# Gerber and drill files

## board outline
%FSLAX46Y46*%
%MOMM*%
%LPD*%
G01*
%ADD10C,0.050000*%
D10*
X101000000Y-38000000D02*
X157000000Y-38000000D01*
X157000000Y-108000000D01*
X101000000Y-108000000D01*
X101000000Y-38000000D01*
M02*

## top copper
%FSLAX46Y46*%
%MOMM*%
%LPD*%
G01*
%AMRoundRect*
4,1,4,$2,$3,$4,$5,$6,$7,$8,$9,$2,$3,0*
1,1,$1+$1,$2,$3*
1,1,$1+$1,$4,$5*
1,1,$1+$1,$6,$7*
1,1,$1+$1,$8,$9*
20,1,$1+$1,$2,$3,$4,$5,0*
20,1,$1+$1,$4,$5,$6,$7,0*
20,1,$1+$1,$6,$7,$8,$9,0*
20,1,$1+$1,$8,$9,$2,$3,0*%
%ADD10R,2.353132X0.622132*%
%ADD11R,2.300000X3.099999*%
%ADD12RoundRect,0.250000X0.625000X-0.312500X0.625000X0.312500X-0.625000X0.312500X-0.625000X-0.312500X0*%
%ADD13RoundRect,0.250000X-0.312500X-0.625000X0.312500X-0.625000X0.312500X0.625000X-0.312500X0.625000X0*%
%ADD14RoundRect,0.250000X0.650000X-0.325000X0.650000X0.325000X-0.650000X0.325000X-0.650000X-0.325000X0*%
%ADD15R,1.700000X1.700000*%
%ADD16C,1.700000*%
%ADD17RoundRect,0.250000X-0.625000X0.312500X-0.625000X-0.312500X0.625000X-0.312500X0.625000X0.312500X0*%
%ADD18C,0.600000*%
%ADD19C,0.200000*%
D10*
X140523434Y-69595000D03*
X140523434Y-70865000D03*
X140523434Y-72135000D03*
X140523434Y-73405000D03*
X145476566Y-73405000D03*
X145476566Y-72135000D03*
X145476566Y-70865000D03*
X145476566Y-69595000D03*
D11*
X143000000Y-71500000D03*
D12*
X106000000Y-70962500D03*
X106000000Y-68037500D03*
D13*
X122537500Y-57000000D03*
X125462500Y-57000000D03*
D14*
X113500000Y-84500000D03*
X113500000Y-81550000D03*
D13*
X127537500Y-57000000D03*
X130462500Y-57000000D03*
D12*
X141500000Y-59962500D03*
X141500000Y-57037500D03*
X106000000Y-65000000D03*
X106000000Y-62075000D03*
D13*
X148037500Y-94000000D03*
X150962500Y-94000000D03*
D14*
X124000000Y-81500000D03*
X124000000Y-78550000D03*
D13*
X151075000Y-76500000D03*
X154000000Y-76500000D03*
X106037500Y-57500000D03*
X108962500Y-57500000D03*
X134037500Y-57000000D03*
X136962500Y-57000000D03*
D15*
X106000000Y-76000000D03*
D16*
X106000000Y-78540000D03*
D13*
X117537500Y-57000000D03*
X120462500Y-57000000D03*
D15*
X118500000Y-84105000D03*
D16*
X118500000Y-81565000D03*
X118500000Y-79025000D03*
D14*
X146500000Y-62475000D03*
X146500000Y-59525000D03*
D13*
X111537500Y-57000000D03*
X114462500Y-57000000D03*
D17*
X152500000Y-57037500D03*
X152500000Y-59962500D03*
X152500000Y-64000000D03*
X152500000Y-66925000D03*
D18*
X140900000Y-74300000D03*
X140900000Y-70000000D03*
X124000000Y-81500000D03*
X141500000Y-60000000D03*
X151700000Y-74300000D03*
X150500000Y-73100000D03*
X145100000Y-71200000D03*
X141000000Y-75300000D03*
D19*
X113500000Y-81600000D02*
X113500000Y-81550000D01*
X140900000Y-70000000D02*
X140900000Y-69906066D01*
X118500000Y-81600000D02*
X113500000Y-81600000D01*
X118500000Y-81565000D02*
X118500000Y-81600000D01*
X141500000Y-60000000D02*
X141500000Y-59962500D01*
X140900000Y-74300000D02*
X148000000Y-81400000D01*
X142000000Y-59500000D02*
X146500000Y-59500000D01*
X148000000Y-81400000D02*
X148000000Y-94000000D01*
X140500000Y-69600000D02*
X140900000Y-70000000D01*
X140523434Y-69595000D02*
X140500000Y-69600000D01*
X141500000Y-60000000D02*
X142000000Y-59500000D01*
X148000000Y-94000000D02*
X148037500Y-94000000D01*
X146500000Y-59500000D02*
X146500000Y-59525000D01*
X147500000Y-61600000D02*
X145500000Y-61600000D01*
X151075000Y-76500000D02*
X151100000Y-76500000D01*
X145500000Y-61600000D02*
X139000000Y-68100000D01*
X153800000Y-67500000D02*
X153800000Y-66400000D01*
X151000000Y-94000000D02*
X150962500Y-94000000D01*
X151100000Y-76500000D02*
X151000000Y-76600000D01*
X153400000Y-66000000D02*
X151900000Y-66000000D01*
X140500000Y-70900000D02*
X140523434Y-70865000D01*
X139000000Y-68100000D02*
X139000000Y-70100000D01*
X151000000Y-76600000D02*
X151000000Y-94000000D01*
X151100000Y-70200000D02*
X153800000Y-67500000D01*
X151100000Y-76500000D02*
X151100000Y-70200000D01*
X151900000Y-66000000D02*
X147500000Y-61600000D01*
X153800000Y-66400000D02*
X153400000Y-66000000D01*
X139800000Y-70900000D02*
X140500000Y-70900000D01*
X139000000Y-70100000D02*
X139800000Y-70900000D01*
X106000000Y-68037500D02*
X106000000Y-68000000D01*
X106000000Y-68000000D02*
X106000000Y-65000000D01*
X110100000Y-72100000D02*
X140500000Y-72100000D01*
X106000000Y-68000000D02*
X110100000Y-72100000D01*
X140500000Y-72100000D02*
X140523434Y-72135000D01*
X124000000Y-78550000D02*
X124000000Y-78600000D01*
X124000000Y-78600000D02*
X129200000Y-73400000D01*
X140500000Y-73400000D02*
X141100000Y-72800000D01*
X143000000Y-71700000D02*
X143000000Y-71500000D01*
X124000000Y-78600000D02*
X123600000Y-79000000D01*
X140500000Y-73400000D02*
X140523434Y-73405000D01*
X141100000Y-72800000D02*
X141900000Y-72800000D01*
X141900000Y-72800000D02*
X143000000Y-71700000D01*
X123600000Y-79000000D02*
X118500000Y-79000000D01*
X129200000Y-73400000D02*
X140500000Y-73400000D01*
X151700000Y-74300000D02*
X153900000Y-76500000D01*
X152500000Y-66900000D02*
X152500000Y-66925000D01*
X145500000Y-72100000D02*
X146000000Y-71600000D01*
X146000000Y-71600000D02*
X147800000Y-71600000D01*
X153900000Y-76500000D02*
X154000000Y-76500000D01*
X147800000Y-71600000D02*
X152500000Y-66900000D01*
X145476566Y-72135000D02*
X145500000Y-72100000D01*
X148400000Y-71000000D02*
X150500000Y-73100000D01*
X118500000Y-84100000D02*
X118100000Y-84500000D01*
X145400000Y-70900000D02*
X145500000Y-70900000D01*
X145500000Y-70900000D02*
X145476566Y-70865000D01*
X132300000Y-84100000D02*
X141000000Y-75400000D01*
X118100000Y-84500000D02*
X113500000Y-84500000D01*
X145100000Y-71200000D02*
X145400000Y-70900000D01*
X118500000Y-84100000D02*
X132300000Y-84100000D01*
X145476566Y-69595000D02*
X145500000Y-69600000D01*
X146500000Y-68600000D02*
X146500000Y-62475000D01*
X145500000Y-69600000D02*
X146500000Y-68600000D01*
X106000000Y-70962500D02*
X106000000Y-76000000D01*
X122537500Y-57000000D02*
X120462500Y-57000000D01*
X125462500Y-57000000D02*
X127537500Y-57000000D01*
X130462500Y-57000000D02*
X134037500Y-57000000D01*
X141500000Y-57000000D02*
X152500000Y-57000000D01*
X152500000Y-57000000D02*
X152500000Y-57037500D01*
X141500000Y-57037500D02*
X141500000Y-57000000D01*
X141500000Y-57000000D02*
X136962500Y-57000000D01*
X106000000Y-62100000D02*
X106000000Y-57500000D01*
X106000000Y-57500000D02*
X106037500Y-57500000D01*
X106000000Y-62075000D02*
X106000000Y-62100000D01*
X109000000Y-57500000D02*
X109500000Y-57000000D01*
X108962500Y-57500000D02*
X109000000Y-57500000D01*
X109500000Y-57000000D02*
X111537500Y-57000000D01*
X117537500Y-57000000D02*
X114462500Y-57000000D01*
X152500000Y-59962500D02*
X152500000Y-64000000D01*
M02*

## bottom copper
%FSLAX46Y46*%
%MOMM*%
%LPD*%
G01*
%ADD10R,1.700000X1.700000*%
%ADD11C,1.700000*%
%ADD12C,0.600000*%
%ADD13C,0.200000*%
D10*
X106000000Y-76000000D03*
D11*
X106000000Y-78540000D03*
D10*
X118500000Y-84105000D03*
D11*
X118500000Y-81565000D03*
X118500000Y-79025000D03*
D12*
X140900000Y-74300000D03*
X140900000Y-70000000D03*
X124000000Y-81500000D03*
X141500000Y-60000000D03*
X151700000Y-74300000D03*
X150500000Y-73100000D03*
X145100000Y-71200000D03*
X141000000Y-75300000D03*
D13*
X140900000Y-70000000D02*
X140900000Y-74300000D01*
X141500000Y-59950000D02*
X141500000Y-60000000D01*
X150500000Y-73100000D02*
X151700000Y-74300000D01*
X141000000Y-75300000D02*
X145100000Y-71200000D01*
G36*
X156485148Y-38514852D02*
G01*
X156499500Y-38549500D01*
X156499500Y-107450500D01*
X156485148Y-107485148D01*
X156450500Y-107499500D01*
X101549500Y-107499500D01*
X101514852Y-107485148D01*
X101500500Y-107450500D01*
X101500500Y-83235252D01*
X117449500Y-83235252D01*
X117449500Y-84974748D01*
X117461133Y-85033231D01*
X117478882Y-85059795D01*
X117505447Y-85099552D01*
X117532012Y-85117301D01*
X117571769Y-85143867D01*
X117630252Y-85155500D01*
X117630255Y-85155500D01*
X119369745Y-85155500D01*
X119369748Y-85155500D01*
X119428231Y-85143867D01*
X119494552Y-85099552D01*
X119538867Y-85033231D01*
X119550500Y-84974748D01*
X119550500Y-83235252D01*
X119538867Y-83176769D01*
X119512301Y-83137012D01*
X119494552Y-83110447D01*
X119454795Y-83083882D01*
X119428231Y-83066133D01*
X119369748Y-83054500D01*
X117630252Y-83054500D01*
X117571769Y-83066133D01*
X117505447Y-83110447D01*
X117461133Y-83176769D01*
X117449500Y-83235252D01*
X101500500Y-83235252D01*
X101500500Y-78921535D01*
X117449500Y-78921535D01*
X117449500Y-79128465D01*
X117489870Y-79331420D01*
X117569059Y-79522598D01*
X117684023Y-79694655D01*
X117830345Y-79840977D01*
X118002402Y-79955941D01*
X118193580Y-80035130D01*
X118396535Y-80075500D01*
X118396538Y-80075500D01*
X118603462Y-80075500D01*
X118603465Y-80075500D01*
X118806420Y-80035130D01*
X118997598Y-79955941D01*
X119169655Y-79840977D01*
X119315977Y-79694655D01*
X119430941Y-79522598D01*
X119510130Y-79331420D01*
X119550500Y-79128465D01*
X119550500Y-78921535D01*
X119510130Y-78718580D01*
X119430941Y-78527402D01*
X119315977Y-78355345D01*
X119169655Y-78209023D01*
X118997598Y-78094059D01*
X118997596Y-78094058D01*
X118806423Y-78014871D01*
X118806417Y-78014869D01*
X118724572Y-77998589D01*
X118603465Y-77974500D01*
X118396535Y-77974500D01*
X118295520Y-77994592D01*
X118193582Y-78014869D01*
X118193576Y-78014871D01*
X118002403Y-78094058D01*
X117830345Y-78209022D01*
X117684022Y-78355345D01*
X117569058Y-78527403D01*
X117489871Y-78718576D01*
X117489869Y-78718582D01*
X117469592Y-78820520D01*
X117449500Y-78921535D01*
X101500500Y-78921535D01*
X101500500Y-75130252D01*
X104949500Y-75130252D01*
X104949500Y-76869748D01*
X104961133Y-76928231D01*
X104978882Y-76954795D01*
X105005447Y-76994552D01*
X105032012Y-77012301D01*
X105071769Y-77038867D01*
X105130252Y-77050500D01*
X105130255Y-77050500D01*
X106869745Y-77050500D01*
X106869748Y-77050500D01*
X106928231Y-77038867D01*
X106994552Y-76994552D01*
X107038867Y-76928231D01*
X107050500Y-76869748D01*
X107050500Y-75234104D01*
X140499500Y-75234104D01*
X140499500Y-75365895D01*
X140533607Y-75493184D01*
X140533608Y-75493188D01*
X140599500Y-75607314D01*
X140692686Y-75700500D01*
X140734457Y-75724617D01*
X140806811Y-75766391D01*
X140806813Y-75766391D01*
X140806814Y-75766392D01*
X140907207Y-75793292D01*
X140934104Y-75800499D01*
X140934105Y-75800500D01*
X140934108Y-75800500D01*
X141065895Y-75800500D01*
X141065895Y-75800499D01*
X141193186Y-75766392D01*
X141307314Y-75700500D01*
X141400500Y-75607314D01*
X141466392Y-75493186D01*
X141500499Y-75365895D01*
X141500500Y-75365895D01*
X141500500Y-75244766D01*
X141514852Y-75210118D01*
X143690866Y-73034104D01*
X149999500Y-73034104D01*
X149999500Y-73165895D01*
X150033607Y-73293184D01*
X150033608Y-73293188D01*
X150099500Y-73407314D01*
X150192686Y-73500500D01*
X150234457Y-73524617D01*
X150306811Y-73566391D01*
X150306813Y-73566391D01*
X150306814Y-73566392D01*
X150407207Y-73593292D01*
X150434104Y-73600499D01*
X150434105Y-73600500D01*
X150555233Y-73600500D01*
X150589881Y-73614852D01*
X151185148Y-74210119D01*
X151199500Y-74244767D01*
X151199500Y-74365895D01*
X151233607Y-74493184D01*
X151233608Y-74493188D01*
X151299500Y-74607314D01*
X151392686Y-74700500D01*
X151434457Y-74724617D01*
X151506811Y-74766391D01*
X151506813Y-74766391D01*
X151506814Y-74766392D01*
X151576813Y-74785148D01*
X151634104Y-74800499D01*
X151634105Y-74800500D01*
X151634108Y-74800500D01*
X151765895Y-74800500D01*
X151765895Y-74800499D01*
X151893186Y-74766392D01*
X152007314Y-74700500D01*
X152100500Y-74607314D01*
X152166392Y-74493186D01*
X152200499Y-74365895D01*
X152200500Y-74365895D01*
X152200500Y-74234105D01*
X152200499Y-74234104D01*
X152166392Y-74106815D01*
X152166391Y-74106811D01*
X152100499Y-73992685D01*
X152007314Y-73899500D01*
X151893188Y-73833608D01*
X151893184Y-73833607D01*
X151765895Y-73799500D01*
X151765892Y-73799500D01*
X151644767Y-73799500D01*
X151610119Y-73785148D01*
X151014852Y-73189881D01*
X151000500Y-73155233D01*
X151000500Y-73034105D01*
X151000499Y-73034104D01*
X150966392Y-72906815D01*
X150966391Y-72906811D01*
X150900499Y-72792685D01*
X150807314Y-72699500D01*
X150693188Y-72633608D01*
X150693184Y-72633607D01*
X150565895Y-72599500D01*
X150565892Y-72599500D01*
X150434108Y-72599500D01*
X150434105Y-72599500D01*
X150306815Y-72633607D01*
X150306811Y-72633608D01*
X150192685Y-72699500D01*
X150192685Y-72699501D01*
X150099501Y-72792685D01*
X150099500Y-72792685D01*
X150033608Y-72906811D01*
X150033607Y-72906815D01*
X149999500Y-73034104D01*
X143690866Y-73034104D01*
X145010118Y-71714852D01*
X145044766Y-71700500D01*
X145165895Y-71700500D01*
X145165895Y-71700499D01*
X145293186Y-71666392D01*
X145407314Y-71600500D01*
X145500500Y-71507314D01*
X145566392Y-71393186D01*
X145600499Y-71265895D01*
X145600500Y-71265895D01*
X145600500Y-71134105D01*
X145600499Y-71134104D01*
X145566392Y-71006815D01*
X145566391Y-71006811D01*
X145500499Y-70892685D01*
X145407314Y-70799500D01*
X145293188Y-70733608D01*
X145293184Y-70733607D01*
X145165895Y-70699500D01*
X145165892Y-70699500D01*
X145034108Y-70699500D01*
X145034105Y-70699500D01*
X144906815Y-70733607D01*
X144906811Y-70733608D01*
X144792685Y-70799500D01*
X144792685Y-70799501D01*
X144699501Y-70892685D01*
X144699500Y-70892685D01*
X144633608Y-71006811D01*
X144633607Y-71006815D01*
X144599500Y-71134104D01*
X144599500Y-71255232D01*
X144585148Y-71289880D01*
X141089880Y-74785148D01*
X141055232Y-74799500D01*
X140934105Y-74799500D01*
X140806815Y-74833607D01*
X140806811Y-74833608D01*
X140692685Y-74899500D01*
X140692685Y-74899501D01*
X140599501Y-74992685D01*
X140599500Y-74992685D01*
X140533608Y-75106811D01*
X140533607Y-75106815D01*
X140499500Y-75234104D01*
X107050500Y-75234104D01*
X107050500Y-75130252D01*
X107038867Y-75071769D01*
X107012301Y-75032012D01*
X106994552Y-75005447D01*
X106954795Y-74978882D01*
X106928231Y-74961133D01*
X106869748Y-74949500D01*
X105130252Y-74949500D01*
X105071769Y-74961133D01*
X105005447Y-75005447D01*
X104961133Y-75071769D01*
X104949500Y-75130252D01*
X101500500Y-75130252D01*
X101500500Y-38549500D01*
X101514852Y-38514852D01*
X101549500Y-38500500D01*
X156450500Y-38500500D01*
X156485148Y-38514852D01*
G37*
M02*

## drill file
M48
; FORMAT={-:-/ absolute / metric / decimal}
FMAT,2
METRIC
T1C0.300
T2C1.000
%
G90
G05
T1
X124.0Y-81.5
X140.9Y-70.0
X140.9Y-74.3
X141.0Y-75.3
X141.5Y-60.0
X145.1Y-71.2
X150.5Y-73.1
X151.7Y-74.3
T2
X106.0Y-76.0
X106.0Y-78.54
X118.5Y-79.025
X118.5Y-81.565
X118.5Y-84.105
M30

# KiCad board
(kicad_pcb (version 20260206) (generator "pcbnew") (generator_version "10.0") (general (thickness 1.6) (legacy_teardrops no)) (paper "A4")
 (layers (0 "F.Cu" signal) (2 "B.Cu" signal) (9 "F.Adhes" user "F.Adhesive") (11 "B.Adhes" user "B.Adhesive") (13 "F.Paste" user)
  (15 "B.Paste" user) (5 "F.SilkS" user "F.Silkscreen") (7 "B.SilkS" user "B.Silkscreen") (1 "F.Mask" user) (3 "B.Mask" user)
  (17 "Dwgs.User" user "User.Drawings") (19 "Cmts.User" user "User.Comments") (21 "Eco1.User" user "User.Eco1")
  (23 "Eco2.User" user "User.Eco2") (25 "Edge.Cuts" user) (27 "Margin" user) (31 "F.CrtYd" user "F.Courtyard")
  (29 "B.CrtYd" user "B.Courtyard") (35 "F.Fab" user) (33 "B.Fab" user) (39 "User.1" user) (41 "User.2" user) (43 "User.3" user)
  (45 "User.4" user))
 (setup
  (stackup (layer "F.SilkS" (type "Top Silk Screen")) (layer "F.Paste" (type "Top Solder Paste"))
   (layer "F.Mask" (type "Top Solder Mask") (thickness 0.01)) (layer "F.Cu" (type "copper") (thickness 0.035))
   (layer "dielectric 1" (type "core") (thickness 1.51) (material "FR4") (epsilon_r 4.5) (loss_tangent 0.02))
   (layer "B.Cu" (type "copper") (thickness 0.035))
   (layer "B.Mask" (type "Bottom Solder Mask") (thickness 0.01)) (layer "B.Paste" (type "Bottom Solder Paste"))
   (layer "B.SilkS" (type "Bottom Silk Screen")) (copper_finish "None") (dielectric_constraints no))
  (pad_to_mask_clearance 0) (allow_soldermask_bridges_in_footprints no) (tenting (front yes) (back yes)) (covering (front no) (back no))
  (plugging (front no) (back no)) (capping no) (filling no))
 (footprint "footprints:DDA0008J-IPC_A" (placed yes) (layer "F.Cu") (at 143 71.5)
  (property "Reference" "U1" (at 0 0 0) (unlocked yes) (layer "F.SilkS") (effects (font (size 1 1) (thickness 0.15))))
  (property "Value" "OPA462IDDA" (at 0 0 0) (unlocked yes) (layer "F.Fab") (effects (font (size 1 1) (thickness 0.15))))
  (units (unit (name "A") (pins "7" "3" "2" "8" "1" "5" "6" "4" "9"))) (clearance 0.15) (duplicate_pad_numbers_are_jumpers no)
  (pad "1" smd rect (at -2.476566 -1.905) (size 2.353132 0.622132) (layers "F.Cu" "F.Mask" "F.Paste") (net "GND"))
  (pad "2" smd rect (at -2.476566 -0.635) (size 2.353132 0.622132) (layers "F.Cu" "F.Mask" "F.Paste") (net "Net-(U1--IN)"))
  (pad "3" smd rect (at -2.476566 0.635) (size 2.353132 0.622132) (layers "F.Cu" "F.Mask" "F.Paste") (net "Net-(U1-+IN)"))
  (pad "4" smd rect (at -2.476566 1.905) (size 2.353132 0.622132) (layers "F.Cu" "F.Mask" "F.Paste") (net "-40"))
  (pad "5" smd rect (at 2.476566 1.905) (size 2.353132 0.622132) (layers "F.Cu" "F.Mask" "F.Paste")
   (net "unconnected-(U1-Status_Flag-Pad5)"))
  (pad "6" smd rect (at 2.476566 0.635) (size 2.353132 0.622132) (layers "F.Cu" "F.Mask" "F.Paste") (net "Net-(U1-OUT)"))
  (pad "7" smd rect (at 2.476566 -0.635) (size 2.353132 0.622132) (layers "F.Cu" "F.Mask" "F.Paste") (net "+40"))
  (pad "8" smd rect (at 2.476566 -1.905) (size 2.353132 0.622132) (layers "F.Cu" "F.Mask" "F.Paste") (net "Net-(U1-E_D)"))
  (pad "9" smd rect (at 0 0) (size 2.3 3.099999) (layers "F.Cu" "F.Mask") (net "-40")))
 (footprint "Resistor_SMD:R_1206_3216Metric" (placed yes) (layer "F.Cu") (at 106 69.5 90)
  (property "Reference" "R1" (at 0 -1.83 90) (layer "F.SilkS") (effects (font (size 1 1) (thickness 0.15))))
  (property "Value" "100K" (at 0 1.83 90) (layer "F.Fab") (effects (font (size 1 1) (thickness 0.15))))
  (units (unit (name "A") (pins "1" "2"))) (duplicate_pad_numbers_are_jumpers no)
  (pad "1" smd roundrect (at -1.4625 0 90) (size 1.125 1.75) (layers "F.Cu" "F.Mask" "F.Paste") (roundrect_rratio 0.222222)
   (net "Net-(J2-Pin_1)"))
  (pad "2" smd roundrect (at 1.4625 0 90) (size 1.125 1.75) (layers "F.Cu" "F.Mask" "F.Paste") (roundrect_rratio 0.222222)
   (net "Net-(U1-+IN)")))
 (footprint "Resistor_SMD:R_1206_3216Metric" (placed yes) (layer "F.Cu") (at 124 57)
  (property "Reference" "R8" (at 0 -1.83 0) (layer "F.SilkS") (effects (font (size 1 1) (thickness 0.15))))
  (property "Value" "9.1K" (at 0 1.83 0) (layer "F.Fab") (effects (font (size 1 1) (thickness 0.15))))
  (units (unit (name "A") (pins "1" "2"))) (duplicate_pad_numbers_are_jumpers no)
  (pad "1" smd roundrect (at -1.4625 0) (size 1.125 1.75) (layers "F.Cu" "F.Mask" "F.Paste") (roundrect_rratio 0.222222)
   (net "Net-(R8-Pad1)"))
  (pad "2" smd roundrect (at 1.4625 0) (size 1.125 1.75) (layers "F.Cu" "F.Mask" "F.Paste") (roundrect_rratio 0.222222)
   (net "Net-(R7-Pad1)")))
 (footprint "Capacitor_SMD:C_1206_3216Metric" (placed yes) (layer "F.Cu") (at 113.5 83.025 90)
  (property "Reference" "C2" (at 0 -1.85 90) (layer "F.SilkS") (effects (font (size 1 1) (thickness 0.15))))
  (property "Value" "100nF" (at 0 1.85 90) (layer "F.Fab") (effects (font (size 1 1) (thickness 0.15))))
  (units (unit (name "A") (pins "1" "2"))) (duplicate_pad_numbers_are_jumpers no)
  (pad "1" smd roundrect (at -1.475 0 90) (size 1.15 1.8) (layers "F.Cu" "F.Mask" "F.Paste") (roundrect_rratio 0.217391) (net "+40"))
  (pad "2" smd roundrect (at 1.475 0 90) (size 1.15 1.8) (layers "F.Cu" "F.Mask" "F.Paste") (roundrect_rratio 0.217391) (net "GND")))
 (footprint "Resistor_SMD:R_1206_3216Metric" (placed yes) (layer "F.Cu") (at 129 57)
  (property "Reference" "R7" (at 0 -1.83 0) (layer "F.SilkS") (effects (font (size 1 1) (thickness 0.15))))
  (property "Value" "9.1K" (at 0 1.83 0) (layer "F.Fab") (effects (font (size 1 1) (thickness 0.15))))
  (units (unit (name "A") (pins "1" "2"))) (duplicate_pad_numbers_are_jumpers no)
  (pad "1" smd roundrect (at -1.4625 0) (size 1.125 1.75) (layers "F.Cu" "F.Mask" "F.Paste") (roundrect_rratio 0.222222)
   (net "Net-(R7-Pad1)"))
  (pad "2" smd roundrect (at 1.4625 0) (size 1.125 1.75) (layers "F.Cu" "F.Mask" "F.Paste") (roundrect_rratio 0.222222)
   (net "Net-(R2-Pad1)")))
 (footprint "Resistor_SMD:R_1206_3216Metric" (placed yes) (layer "F.Cu") (at 141.5 58.5 90)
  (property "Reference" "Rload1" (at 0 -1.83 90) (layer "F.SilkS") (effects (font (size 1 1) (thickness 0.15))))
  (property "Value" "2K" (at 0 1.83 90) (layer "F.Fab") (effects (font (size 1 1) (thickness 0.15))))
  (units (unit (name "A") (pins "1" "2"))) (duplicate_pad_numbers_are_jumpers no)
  (pad "1" smd roundrect (at -1.4625 0 90) (size 1.125 1.75) (layers "F.Cu" "F.Mask" "F.Paste") (roundrect_rratio 0.222222) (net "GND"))
  (pad "2" smd roundrect (at 1.4625 0 90) (size 1.125 1.75) (layers "F.Cu" "F.Mask" "F.Paste") (roundrect_rratio 0.222222)
   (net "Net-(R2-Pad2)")))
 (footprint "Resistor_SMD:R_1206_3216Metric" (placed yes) (layer "F.Cu") (at 106 63.5375 90)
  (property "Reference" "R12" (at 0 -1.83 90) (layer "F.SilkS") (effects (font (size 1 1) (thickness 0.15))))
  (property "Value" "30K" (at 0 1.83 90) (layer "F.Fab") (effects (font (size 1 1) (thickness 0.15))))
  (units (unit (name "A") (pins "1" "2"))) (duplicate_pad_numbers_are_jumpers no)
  (pad "1" smd roundrect (at -1.4625 0 90) (size 1.125 1.75) (layers "F.Cu" "F.Mask" "F.Paste") (roundrect_rratio 0.222222)
   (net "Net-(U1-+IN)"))
  (pad "2" smd roundrect (at 1.4625 0 90) (size 1.125 1.75) (layers "F.Cu" "F.Mask" "F.Paste") (roundrect_rratio 0.222222)
   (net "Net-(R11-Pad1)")))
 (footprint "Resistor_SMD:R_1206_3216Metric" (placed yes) (layer "F.Cu") (at 149.5 94)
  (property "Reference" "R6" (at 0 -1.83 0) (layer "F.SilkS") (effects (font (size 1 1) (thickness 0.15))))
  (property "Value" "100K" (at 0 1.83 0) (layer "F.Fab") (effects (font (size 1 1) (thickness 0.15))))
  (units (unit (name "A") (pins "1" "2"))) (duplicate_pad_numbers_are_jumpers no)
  (pad "1" smd roundrect (at -1.4625 0) (size 1.125 1.75) (layers "F.Cu" "F.Mask" "F.Paste") (roundrect_rratio 0.222222) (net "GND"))
  (pad "2" smd roundrect (at 1.4625 0) (size 1.125 1.75) (layers "F.Cu" "F.Mask" "F.Paste") (roundrect_rratio 0.222222) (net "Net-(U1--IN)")))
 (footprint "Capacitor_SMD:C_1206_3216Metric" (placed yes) (layer "F.Cu") (at 124 80.025 90)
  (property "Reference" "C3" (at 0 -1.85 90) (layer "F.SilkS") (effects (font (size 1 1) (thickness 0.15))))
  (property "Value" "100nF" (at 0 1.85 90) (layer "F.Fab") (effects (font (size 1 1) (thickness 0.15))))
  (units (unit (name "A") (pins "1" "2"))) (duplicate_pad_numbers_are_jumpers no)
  (pad "1" smd roundrect (at -1.475 0 90) (size 1.15 1.8) (layers "F.Cu" "F.Mask" "F.Paste") (roundrect_rratio 0.217391) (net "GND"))
  (pad "2" smd roundrect (at 1.475 0 90) (size 1.15 1.8) (layers "F.Cu" "F.Mask" "F.Paste") (roundrect_rratio 0.217391) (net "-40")))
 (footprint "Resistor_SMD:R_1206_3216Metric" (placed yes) (layer "F.Cu") (at 152.5375 76.5)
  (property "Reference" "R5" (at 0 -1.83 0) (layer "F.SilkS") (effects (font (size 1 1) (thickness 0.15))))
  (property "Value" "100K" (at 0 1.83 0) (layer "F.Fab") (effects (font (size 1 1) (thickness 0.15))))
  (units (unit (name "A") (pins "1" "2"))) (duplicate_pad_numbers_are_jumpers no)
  (pad "1" smd roundrect (at -1.4625 0) (size 1.125 1.75) (layers "F.Cu" "F.Mask" "F.Paste") (roundrect_rratio 0.222222)
   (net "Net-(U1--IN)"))
  (pad "2" smd roundrect (at 1.4625 0) (size 1.125 1.75) (layers "F.Cu" "F.Mask" "F.Paste") (roundrect_rratio 0.222222) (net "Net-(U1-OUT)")))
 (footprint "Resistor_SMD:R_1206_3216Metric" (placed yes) (layer "F.Cu") (at 107.5 57.5)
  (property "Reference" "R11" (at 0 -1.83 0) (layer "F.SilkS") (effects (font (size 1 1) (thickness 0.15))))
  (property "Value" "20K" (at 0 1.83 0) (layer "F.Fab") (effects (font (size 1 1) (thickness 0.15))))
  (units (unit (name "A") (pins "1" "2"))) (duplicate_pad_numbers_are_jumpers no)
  (pad "1" smd roundrect (at -1.4625 0) (size 1.125 1.75) (layers "F.Cu" "F.Mask" "F.Paste") (roundrect_rratio 0.222222)
   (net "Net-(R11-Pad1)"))
  (pad "2" smd roundrect (at 1.4625 0) (size 1.125 1.75) (layers "F.Cu" "F.Mask" "F.Paste") (roundrect_rratio 0.222222)
   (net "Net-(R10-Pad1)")))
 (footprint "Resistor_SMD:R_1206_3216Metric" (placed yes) (layer "F.Cu") (at 135.5 57)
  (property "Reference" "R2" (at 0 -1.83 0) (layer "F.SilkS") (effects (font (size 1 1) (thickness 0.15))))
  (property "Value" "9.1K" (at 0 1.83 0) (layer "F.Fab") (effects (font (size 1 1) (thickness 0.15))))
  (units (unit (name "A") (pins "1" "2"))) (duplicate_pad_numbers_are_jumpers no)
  (pad "1" smd roundrect (at -1.4625 0) (size 1.125 1.75) (layers "F.Cu" "F.Mask" "F.Paste") (roundrect_rratio 0.222222)
   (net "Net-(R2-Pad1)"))
  (pad "2" smd roundrect (at 1.4625 0) (size 1.125 1.75) (layers "F.Cu" "F.Mask" "F.Paste") (roundrect_rratio 0.222222)
   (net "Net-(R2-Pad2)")))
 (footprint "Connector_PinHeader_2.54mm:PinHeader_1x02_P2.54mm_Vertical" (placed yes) (layer "F.Cu") (at 106 76)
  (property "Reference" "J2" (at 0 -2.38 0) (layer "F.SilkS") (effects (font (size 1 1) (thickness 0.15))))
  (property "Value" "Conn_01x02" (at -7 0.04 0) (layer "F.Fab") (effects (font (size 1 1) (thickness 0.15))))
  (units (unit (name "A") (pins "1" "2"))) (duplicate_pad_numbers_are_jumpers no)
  (pad "1" thru_hole rect (at 0 0) (size 1.7 1.7) (drill 1) (layers "*.Cu" "*.Mask") (remove_unused_layers no) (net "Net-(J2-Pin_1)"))
  (pad "2" thru_hole circle (at 0 2.54) (size 1.7 1.7) (drill 1) (layers "*.Cu" "*.Mask") (remove_unused_layers no) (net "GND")))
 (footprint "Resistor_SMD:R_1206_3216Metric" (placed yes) (layer "F.Cu") (at 119 57)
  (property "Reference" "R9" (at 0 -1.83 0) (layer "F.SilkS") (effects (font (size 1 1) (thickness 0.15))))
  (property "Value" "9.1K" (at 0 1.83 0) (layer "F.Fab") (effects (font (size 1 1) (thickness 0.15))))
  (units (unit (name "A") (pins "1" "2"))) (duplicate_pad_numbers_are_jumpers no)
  (pad "1" smd roundrect (at -1.4625 0) (size 1.125 1.75) (layers "F.Cu" "F.Mask" "F.Paste") (roundrect_rratio 0.222222)
   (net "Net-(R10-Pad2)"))
  (pad "2" smd roundrect (at 1.4625 0) (size 1.125 1.75) (layers "F.Cu" "F.Mask" "F.Paste") (roundrect_rratio 0.222222)
   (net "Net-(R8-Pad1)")))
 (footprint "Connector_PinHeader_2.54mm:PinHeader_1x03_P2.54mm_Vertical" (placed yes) (layer "F.Cu") (at 118.5 84.105 180)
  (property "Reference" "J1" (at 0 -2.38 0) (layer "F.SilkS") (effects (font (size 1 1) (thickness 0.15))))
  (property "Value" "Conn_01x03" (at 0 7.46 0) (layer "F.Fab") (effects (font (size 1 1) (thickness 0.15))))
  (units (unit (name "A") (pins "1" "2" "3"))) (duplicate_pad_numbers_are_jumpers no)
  (pad "1" thru_hole rect (at 0 0 180) (size 1.7 1.7) (drill 1) (layers "*.Cu" "*.Mask") (remove_unused_layers no) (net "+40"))
  (pad "2" thru_hole circle (at 0 2.54 180) (size 1.7 1.7) (drill 1) (layers "*.Cu" "*.Mask") (remove_unused_layers no) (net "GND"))
  (pad "3" thru_hole circle (at 0 5.08 180) (size 1.7 1.7) (drill 1) (layers "*.Cu" "*.Mask") (remove_unused_layers no) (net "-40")))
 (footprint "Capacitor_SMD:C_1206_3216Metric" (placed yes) (layer "F.Cu") (at 146.5 61 90)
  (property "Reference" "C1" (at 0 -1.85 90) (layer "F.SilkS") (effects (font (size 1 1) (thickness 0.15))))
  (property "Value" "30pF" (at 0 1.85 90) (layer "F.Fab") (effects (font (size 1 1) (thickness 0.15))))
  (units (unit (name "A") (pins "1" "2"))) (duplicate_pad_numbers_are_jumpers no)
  (pad "1" smd roundrect (at -1.475 0 90) (size 1.15 1.8) (layers "F.Cu" "F.Mask" "F.Paste") (roundrect_rratio 0.217391)
   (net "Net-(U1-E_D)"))
  (pad "2" smd roundrect (at 1.475 0 90) (size 1.15 1.8) (layers "F.Cu" "F.Mask" "F.Paste") (roundrect_rratio 0.217391) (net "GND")))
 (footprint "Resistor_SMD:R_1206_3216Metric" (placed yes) (layer "F.Cu") (at 113 57)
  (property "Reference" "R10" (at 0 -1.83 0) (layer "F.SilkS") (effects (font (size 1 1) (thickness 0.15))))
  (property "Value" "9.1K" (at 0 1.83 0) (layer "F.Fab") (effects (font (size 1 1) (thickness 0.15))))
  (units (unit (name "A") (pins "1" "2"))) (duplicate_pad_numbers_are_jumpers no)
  (pad "1" smd roundrect (at -1.4625 0) (size 1.125 1.75) (layers "F.Cu" "F.Mask" "F.Paste") (roundrect_rratio 0.222222)
   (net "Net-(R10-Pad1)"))
  (pad "2" smd roundrect (at 1.4625 0) (size 1.125 1.75) (layers "F.Cu" "F.Mask" "F.Paste") (roundrect_rratio 0.222222)
   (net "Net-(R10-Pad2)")))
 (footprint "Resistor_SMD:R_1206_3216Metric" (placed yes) (layer "F.Cu") (at 152.5 58.5 -90)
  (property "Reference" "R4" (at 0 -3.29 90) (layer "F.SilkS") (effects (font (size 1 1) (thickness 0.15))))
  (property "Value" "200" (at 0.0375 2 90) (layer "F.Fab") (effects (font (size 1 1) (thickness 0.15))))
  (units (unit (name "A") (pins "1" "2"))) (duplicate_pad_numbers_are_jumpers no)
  (pad "1" smd roundrect (at -1.4625 0 270) (size 1.125 1.75) (layers "F.Cu" "F.Mask" "F.Paste") (roundrect_rratio 0.222222)
   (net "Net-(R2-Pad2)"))
  (pad "2" smd roundrect (at 1.4625 0 270) (size 1.125 1.75) (layers "F.Cu" "F.Mask" "F.Paste") (roundrect_rratio 0.222222)
   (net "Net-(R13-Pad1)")))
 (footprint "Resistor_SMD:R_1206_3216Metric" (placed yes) (layer "F.Cu") (at 152.5 65.4625 -90)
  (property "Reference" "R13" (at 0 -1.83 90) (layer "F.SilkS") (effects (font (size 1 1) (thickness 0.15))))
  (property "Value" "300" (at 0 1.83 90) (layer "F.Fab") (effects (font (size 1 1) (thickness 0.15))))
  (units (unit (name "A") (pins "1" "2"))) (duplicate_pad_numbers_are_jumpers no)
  (pad "1" smd roundrect (at -1.4625 0 270) (size 1.125 1.75) (layers "F.Cu" "F.Mask" "F.Paste") (roundrect_rratio 0.222222)
   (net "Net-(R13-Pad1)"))
  (pad "2" smd roundrect (at 1.4625 0 270) (size 1.125 1.75) (layers "F.Cu" "F.Mask" "F.Paste") (roundrect_rratio 0.222222)
   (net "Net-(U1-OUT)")))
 (gr_rect (start 101 38) (end 157 108) (stroke (width 0.05) (type default)) (fill no) (layer "Edge.Cuts"))
 (segment (start 113.5 81.6) (end 113.5 81.55) (width 0.2) (layer "F.Cu") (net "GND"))
 (segment (start 140.9 70) (end 140.9 69.906066) (width 0.2) (layer "F.Cu") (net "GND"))
 (segment (start 118.5 81.6) (end 113.5 81.6) (width 0.2) (layer "F.Cu") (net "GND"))
 (segment (start 118.5 81.565) (end 118.5 81.6) (width 0.2) (layer "F.Cu") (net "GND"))
 (segment (start 141.5 60) (end 141.5 59.9625) (width 0.2) (layer "F.Cu") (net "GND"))
 (segment (start 140.9 74.3) (end 148 81.4) (width 0.2) (layer "F.Cu") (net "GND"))
 (segment (start 142 59.5) (end 146.5 59.5) (width 0.2) (layer "F.Cu") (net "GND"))
 (segment (start 148 81.4) (end 148 94) (width 0.2) (layer "F.Cu") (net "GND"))
 (segment (start 140.5 69.6) (end 140.9 70) (width 0.2) (layer "F.Cu") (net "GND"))
 (segment (start 140.523434 69.595) (end 140.5 69.6) (width 0.2) (layer "F.Cu") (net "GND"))
 (segment (start 141.5 60) (end 142 59.5) (width 0.2) (layer "F.Cu") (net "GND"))
 (segment (start 148 94) (end 148.0375 94) (width 0.2) (layer "F.Cu") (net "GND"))
 (segment (start 146.5 59.5) (end 146.5 59.525) (width 0.2) (layer "F.Cu") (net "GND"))
 (via (at 140.9 74.3) (size 0.6) (drill 0.3) (layers "F.Cu" "B.Cu") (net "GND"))
 (via (at 140.9 70) (size 0.6) (drill 0.3) (layers "F.Cu" "B.Cu") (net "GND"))
 (via (at 124 81.5) (size 0.6) (drill 0.3) (layers "F.Cu" "B.Cu") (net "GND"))
 (via (at 141.5 60) (size 0.6) (drill 0.3) (layers "F.Cu" "B.Cu") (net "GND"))
 (segment (start 140.9 70) (end 140.9 74.3) (width 0.2) (layer "B.Cu") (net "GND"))
 (segment (start 141.5 59.95) (end 141.5 60) (width 0.2) (layer "B.Cu") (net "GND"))
 (segment (start 147.5 61.6) (end 145.5 61.6) (width 0.2) (layer "F.Cu") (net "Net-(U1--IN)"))
 (segment (start 151.075 76.5) (end 151.1 76.5) (width 0.2) (layer "F.Cu") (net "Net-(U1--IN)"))
 (segment (start 145.5 61.6) (end 139 68.1) (width 0.2) (layer "F.Cu") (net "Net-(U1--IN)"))
 (segment (start 153.8 67.5) (end 153.8 66.4) (width 0.2) (layer "F.Cu") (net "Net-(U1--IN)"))
 (segment (start 151 94) (end 150.9625 94) (width 0.2) (layer "F.Cu") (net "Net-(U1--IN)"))
 (segment (start 151.1 76.5) (end 151 76.6) (width 0.2) (layer "F.Cu") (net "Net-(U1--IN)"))
 (segment (start 153.4 66) (end 151.9 66) (width 0.2) (layer "F.Cu") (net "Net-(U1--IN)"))
 (segment (start 140.5 70.9) (end 140.523434 70.865) (width 0.2) (layer "F.Cu") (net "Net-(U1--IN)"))
 (segment (start 139 68.1) (end 139 70.1) (width 0.2) (layer "F.Cu") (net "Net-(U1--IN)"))
 (segment (start 151 76.6) (end 151 94) (width 0.2) (layer "F.Cu") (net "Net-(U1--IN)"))
 (segment (start 151.1 70.2) (end 153.8 67.5) (width 0.2) (layer "F.Cu") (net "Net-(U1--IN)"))
 (segment (start 151.1 76.5) (end 151.1 70.2) (width 0.2) (layer "F.Cu") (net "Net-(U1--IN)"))
 (segment (start 151.9 66) (end 147.5 61.6) (width 0.2) (layer "F.Cu") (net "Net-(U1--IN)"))
 (segment (start 153.8 66.4) (end 153.4 66) (width 0.2) (layer "F.Cu") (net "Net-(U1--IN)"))
 (segment (start 139.8 70.9) (end 140.5 70.9) (width 0.2) (layer "F.Cu") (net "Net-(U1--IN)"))
 (segment (start 139 70.1) (end 139.8 70.9) (width 0.2) (layer "F.Cu") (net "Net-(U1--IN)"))
 (segment (start 106 68.0375) (end 106 68) (width 0.2) (layer "F.Cu") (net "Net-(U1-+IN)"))
 (segment (start 106 68) (end 106 65) (width 0.2) (layer "F.Cu") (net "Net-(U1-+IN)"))
 (segment (start 110.1 72.1) (end 140.5 72.1) (width 0.2) (layer "F.Cu") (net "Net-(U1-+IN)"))
 (segment (start 106 68) (end 110.1 72.1) (width 0.2) (layer "F.Cu") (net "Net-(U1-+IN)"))
 (segment (start 140.5 72.1) (end 140.523434 72.135) (width 0.2) (layer "F.Cu") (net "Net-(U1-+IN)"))
 (segment (start 124 78.55) (end 124 78.6) (width 0.2) (layer "F.Cu") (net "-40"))
 (segment (start 124 78.6) (end 129.2 73.4) (width 0.2) (layer "F.Cu") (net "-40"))
 (segment (start 140.5 73.4) (end 141.1 72.8) (width 0.2) (layer "F.Cu") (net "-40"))
 (segment (start 143 71.7) (end 143 71.5) (width 0.2) (layer "F.Cu") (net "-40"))
 (segment (start 124 78.6) (end 123.6 79) (width 0.2) (layer "F.Cu") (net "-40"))
 (segment (start 140.5 73.4) (end 140.523434 73.405) (width 0.2) (layer "F.Cu") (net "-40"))
 (segment (start 141.1 72.8) (end 141.9 72.8) (width 0.2) (layer "F.Cu") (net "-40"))
 (segment (start 141.9 72.8) (end 143 71.7) (width 0.2) (layer "F.Cu") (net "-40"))
 (segment (start 123.6 79) (end 118.5 79) (width 0.2) (layer "F.Cu") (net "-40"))
 (segment (start 129.2 73.4) (end 140.5 73.4) (width 0.2) (layer "F.Cu") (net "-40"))
 (segment (start 151.7 74.3) (end 153.9 76.5) (width 0.2) (layer "F.Cu") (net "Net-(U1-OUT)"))
 (segment (start 152.5 66.9) (end 152.5 66.925) (width 0.2) (layer "F.Cu") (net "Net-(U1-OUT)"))
 (segment (start 145.5 72.1) (end 146 71.6) (width 0.2) (layer "F.Cu") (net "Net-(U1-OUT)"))
 (segment (start 146 71.6) (end 147.8 71.6) (width 0.2) (layer "F.Cu") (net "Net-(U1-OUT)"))
 (segment (start 153.9 76.5) (end 154 76.5) (width 0.2) (layer "F.Cu") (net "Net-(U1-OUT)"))
 (segment (start 147.8 71.6) (end 152.5 66.9) (width 0.2) (layer "F.Cu") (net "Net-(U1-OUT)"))
 (segment (start 145.476566 72.135) (end 145.5 72.1) (width 0.2) (layer "F.Cu") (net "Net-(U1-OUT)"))
 (segment (start 148.4 71) (end 150.5 73.1) (width 0.2) (layer "F.Cu") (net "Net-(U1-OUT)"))
 (via (at 151.7 74.3) (size 0.6) (drill 0.3) (layers "F.Cu" "B.Cu") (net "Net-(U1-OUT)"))
 (via (at 150.5 73.1) (size 0.6) (drill 0.3) (layers "F.Cu" "B.Cu") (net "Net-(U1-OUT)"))
 (segment (start 150.5 73.1) (end 151.7 74.3) (width 0.2) (layer "B.Cu") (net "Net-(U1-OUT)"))
 (segment (start 118.5 84.1) (end 118.1 84.5) (width 0.2) (layer "F.Cu") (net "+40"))
 (segment (start 145.4 70.9) (end 145.5 70.9) (width 0.2) (layer "F.Cu") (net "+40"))
 (segment (start 145.5 70.9) (end 145.476566 70.865) (width 0.2) (layer "F.Cu") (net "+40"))
 (segment (start 132.3 84.1) (end 141 75.4) (width 0.2) (layer "F.Cu") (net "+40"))
 (segment (start 118.1 84.5) (end 113.5 84.5) (width 0.2) (layer "F.Cu") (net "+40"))
 (segment (start 145.1 71.2) (end 145.4 70.9) (width 0.2) (layer "F.Cu") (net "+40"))
 (segment (start 118.5 84.1) (end 132.3 84.1) (width 0.2) (layer "F.Cu") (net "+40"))
 (via (at 145.1 71.2) (size 0.6) (drill 0.3) (layers "F.Cu" "B.Cu") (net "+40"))
 (via (at 141 75.3) (size 0.6) (drill 0.3) (layers "F.Cu" "B.Cu") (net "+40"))
 (segment (start 141 75.3) (end 145.1 71.2) (width 0.2) (layer "B.Cu") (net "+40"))
 (segment (start 145.476566 69.595) (end 145.5 69.6) (width 0.2) (layer "F.Cu") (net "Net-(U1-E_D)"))
 (segment (start 146.5 68.6) (end 146.5 62.475) (width 0.2) (layer "F.Cu") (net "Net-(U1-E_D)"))
 (segment (start 145.5 69.6) (end 146.5 68.6) (width 0.2) (layer "F.Cu") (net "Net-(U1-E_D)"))
 (segment (start 106 70.9625) (end 106 76) (width 0.2) (layer "F.Cu") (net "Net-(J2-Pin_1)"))
 (segment (start 122.5375 57) (end 120.4625 57) (width 0.2) (layer "F.Cu") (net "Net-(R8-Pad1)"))
 (segment (start 125.4625 57) (end 127.5375 57) (width 0.2) (layer "F.Cu") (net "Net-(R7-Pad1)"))
 (segment (start 130.4625 57) (end 134.0375 57) (width 0.2) (layer "F.Cu") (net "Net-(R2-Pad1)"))
 (segment (start 141.5 57) (end 152.5 57) (width 0.2) (layer "F.Cu") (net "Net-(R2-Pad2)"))
 (segment (start 152.5 57) (end 152.5 57.0375) (width 0.2) (layer "F.Cu") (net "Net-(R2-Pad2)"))
 (segment (start 141.5 57.0375) (end 141.5 57) (width 0.2) (layer "F.Cu") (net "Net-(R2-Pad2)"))
 (segment (start 141.5 57) (end 136.9625 57) (width 0.2) (layer "F.Cu") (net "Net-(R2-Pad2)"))
 (segment (start 106 62.1) (end 106 57.5) (width 0.2) (layer "F.Cu") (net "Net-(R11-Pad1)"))
 (segment (start 106 57.5) (end 106.0375 57.5) (width 0.2) (layer "F.Cu") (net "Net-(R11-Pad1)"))
 (segment (start 106 62.075) (end 106 62.1) (width 0.2) (layer "F.Cu") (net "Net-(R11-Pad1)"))
 (segment (start 109 57.5) (end 109.5 57) (width 0.2) (layer "F.Cu") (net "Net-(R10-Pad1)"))
 (segment (start 108.9625 57.5) (end 109 57.5) (width 0.2) (layer "F.Cu") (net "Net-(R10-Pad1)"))
 (segment (start 109.5 57) (end 111.5375 57) (width 0.2) (layer "F.Cu") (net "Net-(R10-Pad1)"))
 (segment (start 117.5375 57) (end 114.4625 57) (width 0.2) (layer "F.Cu") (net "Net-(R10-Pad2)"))
 (segment (start 152.5 59.9625) (end 152.5 64) (width 0.2) (layer "F.Cu") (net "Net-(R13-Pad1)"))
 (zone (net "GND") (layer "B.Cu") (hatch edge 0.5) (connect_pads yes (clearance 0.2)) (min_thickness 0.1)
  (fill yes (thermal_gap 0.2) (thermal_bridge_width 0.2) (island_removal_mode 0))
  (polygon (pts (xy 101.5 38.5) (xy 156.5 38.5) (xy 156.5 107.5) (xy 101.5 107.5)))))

